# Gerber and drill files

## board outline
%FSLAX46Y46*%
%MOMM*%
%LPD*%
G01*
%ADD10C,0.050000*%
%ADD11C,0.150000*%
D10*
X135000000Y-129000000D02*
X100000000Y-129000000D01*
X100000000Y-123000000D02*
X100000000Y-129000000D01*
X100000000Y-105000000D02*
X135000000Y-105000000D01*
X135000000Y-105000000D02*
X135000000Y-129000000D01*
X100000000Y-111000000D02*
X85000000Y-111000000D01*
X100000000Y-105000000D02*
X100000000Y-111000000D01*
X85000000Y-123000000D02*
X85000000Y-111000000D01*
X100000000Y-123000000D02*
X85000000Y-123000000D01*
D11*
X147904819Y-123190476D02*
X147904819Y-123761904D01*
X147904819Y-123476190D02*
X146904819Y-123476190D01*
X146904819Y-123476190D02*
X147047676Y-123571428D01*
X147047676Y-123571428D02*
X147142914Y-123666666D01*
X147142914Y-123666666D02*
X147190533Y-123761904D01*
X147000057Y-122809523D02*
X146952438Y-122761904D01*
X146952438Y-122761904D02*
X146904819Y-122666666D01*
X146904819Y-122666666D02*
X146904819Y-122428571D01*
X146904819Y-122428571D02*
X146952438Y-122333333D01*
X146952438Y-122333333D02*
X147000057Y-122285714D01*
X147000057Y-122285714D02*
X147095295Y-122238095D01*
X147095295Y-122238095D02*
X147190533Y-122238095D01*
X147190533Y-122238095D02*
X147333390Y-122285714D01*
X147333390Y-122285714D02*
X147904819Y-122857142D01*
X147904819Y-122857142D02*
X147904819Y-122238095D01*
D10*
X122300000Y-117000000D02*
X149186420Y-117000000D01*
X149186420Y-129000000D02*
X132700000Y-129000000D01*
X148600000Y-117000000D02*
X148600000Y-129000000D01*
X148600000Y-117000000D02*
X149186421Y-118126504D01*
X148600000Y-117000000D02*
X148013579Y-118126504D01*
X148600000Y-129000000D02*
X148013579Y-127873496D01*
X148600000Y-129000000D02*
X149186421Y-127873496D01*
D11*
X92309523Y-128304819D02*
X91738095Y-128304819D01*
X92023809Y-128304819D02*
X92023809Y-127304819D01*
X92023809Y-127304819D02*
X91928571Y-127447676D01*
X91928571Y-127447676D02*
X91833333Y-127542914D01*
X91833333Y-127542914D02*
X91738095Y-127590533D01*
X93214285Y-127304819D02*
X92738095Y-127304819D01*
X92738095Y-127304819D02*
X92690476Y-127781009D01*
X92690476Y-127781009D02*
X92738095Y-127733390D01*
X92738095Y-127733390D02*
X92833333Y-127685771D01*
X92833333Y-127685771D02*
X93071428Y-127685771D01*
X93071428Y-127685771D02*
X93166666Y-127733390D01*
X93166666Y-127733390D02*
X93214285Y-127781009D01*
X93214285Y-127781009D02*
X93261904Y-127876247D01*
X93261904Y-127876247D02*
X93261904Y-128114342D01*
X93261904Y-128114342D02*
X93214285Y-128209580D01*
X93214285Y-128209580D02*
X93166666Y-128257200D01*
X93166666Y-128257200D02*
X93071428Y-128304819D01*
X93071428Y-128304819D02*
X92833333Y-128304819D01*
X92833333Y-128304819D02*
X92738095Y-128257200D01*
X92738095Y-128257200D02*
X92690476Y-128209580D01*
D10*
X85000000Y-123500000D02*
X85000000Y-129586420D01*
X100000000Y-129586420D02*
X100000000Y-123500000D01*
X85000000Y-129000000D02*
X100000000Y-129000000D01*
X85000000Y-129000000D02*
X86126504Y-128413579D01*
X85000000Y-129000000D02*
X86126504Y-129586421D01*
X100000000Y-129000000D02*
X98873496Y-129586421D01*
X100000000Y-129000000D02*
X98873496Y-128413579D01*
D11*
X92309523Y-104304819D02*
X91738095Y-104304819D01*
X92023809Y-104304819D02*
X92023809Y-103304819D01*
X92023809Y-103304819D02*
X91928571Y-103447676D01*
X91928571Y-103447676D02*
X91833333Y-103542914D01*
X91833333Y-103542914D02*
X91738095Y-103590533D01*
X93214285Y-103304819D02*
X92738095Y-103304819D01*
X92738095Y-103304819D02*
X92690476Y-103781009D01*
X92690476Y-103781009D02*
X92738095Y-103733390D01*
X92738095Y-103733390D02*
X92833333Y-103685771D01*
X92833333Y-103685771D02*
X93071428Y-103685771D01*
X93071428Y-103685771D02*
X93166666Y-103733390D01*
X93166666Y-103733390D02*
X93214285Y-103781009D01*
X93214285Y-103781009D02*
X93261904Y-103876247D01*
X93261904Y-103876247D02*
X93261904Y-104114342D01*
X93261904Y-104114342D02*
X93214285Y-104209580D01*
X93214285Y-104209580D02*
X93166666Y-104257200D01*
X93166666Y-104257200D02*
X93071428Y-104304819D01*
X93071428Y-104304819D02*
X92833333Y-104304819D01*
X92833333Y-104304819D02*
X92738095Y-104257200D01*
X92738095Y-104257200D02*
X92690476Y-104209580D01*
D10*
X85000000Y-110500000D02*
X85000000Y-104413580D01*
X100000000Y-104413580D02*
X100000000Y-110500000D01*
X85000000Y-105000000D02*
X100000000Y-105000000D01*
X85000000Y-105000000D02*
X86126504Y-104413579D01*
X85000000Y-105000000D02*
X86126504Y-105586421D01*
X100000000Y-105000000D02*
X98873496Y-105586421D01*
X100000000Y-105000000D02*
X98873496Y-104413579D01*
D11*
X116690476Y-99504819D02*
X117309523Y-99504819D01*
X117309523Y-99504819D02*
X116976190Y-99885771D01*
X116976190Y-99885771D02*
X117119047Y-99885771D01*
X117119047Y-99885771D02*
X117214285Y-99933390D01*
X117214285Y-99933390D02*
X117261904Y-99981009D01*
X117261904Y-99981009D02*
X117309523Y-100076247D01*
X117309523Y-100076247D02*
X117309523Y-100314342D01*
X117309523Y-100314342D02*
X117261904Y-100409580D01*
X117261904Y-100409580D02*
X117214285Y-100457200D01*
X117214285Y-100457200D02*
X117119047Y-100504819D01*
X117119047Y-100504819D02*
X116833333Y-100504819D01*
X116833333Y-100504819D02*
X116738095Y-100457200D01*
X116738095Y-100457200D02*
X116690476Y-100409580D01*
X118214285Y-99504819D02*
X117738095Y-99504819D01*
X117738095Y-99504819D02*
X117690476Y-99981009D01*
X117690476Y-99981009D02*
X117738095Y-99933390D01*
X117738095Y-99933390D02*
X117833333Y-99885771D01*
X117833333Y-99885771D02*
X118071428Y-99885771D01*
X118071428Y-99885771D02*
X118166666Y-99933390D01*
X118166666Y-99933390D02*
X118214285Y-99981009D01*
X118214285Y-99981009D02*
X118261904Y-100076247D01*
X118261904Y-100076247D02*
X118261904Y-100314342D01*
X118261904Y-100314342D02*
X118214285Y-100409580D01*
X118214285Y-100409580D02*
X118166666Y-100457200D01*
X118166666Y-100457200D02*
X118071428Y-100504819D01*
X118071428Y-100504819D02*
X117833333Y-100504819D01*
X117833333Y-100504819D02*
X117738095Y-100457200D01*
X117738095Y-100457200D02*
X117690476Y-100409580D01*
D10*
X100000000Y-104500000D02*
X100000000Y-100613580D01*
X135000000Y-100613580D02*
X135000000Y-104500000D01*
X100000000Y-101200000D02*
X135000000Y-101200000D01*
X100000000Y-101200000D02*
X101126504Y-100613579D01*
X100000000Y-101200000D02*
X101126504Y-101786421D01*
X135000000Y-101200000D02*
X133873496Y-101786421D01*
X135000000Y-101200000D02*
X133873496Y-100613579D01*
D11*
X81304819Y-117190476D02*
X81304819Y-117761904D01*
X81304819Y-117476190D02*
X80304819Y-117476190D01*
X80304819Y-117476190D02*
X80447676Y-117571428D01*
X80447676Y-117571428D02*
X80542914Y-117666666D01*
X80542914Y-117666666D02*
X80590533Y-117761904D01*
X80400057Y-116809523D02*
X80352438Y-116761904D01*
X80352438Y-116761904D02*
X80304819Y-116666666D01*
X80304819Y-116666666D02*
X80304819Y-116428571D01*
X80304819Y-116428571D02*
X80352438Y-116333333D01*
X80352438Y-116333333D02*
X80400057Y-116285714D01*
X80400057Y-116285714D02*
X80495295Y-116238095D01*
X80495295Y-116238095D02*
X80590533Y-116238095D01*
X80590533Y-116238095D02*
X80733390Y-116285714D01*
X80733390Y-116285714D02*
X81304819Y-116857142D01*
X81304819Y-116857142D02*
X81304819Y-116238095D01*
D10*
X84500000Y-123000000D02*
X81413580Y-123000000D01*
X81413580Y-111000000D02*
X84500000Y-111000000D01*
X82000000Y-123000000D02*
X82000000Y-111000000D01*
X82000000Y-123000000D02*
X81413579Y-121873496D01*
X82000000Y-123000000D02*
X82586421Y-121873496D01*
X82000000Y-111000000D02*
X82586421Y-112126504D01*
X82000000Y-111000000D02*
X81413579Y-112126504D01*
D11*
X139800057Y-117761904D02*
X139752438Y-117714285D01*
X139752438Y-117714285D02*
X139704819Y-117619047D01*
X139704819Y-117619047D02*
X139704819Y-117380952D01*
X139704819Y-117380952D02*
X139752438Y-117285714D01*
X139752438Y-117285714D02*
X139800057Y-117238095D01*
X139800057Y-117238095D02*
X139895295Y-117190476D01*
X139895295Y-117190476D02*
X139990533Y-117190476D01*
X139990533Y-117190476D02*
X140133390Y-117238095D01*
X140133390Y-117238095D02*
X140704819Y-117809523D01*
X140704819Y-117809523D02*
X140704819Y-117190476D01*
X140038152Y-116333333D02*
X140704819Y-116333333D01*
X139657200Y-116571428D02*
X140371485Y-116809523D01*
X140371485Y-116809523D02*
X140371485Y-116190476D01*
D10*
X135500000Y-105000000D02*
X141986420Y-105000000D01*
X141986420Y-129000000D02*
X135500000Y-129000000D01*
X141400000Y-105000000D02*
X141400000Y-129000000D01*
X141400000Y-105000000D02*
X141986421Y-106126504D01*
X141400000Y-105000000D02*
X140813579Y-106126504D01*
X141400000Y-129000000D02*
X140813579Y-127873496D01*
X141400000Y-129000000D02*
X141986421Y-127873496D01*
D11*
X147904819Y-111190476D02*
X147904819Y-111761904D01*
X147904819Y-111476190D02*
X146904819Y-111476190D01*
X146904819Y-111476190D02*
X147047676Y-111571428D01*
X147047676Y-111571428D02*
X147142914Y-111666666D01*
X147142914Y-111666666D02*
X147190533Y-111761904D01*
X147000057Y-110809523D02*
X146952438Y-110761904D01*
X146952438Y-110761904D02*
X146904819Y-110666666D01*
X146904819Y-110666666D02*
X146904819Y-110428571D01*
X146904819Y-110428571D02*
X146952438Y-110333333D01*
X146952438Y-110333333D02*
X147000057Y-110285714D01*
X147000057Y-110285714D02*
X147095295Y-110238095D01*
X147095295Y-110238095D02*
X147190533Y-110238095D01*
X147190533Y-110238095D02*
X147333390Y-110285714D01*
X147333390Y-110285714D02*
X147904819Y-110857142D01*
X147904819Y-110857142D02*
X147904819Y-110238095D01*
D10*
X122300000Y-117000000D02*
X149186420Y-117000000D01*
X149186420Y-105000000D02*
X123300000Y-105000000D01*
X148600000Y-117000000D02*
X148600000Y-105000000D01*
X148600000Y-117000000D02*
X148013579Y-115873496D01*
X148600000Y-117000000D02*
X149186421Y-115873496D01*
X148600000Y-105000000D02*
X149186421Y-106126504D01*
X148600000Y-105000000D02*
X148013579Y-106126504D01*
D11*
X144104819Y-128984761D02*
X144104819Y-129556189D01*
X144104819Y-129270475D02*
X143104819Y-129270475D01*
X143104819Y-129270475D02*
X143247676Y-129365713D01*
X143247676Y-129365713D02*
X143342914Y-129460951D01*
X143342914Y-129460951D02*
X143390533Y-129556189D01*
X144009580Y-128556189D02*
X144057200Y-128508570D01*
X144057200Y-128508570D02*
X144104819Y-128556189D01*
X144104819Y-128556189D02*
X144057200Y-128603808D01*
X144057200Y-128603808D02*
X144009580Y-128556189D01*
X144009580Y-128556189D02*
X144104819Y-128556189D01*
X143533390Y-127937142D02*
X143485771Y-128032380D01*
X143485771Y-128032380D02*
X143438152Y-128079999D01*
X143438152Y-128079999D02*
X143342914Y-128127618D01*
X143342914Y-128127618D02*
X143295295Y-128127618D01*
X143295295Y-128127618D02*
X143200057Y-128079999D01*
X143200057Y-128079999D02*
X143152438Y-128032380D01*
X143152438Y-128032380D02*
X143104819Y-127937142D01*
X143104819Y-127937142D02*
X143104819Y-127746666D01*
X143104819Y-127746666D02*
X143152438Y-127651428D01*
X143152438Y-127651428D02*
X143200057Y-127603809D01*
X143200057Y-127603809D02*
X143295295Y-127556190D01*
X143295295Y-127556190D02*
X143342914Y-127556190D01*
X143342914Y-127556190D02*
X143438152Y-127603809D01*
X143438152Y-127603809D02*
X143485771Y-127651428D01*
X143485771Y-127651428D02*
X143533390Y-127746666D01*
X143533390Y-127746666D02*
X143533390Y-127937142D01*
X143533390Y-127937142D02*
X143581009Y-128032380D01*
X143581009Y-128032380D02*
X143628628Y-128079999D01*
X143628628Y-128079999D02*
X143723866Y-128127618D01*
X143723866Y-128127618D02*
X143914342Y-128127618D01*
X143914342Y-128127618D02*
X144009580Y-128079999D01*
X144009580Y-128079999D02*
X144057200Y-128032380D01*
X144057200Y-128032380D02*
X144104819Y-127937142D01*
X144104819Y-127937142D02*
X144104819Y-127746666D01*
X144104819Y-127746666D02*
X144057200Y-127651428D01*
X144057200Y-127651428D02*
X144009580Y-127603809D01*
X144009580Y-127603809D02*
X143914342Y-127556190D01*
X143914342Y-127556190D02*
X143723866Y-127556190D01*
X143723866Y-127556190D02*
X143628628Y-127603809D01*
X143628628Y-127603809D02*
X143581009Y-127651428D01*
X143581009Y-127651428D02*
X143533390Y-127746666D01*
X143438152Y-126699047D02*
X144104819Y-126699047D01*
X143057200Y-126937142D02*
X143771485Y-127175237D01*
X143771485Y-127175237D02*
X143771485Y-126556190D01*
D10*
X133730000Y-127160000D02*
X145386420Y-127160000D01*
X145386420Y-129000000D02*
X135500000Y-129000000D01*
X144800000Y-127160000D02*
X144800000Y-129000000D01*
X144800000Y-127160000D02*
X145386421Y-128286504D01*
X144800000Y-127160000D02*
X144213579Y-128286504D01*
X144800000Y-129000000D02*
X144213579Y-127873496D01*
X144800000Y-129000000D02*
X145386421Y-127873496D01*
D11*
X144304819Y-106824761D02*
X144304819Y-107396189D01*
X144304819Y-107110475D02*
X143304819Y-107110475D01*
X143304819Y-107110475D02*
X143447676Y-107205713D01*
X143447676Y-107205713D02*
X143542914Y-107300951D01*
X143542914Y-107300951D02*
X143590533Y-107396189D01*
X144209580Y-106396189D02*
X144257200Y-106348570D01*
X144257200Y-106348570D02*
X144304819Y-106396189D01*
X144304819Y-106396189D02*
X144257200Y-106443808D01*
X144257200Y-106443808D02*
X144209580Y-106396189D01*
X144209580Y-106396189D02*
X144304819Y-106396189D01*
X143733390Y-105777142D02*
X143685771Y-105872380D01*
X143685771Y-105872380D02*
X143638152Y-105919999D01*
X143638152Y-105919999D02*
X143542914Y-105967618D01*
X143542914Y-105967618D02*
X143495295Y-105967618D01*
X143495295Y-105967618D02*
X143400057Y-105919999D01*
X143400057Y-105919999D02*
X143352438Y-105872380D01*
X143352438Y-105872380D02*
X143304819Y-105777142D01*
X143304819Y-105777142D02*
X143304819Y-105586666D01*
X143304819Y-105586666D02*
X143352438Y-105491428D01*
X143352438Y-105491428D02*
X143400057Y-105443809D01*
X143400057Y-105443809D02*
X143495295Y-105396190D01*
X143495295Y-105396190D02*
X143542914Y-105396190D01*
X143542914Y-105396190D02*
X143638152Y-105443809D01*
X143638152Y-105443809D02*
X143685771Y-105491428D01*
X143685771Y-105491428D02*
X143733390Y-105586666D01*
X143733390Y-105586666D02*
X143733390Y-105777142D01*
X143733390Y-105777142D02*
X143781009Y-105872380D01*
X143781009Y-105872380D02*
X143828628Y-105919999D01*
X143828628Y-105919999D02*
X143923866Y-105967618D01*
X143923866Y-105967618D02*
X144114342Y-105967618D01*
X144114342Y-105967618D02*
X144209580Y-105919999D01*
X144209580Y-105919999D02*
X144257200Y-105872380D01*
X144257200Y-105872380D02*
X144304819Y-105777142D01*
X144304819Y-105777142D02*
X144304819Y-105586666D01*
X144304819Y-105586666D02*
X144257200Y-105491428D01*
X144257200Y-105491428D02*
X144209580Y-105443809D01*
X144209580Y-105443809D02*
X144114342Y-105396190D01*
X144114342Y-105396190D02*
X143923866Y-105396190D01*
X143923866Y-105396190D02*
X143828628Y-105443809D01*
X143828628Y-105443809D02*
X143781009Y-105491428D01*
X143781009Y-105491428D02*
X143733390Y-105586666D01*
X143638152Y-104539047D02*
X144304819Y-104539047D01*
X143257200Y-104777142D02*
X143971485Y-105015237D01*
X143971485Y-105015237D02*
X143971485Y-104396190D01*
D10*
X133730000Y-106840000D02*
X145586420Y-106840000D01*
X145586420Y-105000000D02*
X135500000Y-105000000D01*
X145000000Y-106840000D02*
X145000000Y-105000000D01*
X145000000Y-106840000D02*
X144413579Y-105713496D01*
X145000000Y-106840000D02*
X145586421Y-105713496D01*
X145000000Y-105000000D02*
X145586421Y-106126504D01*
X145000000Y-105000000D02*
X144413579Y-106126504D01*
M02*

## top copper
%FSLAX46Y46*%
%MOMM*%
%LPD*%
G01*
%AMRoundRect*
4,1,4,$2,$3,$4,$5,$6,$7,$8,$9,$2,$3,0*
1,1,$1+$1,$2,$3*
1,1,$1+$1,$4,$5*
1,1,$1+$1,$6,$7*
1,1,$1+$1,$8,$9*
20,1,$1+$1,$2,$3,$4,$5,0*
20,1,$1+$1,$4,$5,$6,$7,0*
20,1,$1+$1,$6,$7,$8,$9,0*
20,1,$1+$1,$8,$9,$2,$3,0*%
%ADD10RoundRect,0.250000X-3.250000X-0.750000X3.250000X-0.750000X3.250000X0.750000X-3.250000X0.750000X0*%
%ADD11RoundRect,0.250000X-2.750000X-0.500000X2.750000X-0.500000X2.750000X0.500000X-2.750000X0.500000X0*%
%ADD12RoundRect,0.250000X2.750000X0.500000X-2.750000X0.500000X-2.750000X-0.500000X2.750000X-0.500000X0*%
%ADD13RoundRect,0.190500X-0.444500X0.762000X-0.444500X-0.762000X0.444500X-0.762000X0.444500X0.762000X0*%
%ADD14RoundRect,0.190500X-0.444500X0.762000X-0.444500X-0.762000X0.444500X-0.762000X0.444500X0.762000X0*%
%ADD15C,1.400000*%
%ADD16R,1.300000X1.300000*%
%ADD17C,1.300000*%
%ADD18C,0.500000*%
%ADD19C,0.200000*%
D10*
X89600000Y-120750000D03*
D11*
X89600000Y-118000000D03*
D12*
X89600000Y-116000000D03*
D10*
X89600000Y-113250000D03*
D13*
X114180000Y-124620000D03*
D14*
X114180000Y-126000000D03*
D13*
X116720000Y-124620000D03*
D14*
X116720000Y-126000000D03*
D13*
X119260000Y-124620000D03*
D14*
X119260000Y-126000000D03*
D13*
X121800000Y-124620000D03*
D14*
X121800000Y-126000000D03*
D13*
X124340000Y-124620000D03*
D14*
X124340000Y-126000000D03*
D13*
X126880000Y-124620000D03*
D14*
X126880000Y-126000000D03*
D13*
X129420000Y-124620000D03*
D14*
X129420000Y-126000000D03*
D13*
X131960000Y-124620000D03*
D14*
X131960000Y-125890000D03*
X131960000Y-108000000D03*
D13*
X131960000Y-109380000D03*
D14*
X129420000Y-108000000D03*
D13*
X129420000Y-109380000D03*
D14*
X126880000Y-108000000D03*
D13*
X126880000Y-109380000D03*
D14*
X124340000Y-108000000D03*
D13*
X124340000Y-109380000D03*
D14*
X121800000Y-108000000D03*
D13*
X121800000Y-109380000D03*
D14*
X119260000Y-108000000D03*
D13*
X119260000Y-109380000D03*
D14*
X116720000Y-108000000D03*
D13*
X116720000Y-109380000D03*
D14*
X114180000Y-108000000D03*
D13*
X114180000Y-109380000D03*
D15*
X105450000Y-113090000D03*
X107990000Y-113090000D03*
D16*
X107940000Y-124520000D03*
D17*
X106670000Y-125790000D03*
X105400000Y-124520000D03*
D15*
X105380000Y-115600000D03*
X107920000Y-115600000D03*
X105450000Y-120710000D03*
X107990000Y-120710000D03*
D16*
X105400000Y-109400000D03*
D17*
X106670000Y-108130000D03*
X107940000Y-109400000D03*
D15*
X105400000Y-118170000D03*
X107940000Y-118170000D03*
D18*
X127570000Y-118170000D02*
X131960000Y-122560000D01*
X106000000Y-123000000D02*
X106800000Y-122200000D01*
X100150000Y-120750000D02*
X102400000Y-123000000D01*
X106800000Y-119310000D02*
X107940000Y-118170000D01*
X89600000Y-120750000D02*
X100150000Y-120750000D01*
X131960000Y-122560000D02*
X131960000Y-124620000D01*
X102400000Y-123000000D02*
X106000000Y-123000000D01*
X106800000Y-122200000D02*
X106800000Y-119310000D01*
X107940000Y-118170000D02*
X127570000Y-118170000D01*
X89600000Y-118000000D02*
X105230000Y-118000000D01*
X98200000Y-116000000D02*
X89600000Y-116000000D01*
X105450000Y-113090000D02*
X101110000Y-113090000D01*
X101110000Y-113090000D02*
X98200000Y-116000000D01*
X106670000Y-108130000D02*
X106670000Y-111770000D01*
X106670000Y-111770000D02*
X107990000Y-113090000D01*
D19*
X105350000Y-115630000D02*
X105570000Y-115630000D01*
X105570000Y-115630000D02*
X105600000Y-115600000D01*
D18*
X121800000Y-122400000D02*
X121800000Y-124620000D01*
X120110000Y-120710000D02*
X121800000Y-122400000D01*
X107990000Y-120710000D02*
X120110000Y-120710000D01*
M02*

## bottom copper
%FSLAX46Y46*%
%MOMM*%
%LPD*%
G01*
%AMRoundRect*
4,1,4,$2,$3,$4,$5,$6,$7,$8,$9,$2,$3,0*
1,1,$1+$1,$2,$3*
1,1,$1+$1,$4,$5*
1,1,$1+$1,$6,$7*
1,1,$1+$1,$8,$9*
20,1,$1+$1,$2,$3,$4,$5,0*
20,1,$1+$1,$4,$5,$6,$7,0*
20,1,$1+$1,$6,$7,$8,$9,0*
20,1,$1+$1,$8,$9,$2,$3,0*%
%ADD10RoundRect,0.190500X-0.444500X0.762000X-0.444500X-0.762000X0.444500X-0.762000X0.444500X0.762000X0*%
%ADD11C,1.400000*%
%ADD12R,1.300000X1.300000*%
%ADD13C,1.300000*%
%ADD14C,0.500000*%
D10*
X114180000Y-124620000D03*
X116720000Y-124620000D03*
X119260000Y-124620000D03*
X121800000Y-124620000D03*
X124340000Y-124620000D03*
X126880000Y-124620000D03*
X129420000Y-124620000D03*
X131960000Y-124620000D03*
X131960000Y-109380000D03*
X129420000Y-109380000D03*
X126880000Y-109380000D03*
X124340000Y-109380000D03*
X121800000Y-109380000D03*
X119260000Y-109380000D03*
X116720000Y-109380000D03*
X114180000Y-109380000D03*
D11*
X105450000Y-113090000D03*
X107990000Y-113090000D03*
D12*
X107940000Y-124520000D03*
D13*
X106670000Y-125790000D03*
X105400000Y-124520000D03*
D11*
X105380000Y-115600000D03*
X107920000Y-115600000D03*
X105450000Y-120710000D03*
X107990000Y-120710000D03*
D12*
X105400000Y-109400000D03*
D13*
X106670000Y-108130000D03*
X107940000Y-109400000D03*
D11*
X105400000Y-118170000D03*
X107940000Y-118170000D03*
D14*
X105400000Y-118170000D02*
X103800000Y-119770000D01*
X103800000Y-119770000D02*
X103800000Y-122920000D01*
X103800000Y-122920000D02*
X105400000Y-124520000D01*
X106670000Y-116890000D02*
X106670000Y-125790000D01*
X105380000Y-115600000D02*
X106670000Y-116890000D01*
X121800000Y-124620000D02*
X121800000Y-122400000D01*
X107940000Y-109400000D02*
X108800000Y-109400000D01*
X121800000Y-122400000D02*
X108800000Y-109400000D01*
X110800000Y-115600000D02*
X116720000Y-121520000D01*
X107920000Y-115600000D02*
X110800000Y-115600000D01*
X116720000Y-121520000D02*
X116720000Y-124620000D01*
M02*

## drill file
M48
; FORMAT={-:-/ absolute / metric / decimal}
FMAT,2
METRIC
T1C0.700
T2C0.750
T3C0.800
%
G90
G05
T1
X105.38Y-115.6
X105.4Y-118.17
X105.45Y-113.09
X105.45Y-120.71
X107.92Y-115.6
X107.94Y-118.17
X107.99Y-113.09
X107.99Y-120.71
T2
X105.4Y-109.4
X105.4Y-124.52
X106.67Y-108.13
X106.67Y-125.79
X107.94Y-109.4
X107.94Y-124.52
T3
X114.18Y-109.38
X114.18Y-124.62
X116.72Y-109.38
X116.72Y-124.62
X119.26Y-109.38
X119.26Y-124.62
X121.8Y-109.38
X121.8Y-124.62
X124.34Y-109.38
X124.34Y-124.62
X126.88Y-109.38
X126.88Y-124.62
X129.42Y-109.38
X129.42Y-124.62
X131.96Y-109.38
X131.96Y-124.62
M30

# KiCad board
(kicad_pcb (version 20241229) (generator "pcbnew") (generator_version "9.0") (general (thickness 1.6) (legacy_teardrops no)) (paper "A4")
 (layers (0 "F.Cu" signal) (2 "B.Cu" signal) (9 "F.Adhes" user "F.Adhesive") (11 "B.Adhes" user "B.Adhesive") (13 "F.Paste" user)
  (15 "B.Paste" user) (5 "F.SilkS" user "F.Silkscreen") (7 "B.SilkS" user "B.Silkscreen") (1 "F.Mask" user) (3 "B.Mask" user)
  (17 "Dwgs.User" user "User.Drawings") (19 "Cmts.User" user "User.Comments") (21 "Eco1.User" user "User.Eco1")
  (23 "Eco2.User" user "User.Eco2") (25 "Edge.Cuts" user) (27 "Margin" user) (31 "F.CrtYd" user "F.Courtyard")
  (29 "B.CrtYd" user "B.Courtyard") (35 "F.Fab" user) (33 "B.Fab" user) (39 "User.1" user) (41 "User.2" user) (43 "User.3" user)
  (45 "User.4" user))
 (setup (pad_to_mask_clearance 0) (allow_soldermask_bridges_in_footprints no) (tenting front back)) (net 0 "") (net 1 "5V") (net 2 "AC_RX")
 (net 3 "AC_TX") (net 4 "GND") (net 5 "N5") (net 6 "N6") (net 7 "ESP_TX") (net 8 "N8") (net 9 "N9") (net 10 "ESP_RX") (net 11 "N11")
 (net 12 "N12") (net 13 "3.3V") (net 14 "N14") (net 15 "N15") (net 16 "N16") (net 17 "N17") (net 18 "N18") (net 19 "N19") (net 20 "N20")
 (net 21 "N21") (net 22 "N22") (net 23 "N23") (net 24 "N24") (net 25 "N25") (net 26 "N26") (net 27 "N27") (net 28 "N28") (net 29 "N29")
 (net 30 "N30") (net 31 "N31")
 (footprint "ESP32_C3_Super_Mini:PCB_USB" (layer "F.Cu") (at 89.6 117)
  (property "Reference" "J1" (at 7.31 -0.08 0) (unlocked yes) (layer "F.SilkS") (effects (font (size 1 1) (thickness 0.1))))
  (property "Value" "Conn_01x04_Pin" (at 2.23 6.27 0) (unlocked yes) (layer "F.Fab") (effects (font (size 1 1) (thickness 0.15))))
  (pad "1" smd roundrect (at 0 3.75) (size 7 2) (layers "F.Cu" "F.Mask" "F.Paste") (roundrect_rratio 0.125) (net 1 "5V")
   (thermal_bridge_angle 45))
  (pad "2" smd roundrect (at 0 1) (size 6 1.5) (layers "F.Cu" "F.Mask" "F.Paste") (roundrect_rratio 0.1666666667) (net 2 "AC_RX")
   (thermal_bridge_angle 45))
  (pad "3" smd roundrect (at 0 -1 180) (size 6 1.5) (layers "F.Cu" "F.Mask" "F.Paste") (roundrect_rratio 0.1666666667) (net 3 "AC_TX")
   (thermal_bridge_angle 45))
  (pad "4" smd roundrect (at 0 -3.75) (size 7 2) (layers "F.Cu" "F.Mask" "F.Paste") (roundrect_rratio 0.125) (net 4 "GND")
   (thermal_bridge_angle 45)))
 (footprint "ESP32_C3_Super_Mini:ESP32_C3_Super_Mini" (layer "F.Cu") (at 121.8 117 -90)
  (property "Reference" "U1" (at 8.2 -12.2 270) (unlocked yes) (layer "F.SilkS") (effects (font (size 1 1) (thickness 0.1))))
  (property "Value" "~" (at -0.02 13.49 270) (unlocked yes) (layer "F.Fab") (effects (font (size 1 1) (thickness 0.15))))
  (pad "0" thru_hole roundrect (at 7.62 7.62 270) (size 1.905 1.27) (drill 0.8) (layers "*.Cu" "*.Mask") (remove_unused_layers no)
   (roundrect_rratio 0.15) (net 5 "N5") (thermal_bridge_angle 45))
  (pad "0" smd roundrect (at 9 7.62 270) (size 1.905 1.27) (layers "F.Cu" "F.Mask" "F.Paste") (roundrect_rratio 0.15) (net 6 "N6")
   (thermal_bridge_angle 45))
  (pad "1" thru_hole roundrect (at 7.62 5.08 270) (size 1.905 1.27) (drill 0.8) (layers "*.Cu" "*.Mask") (remove_unused_layers no)
   (roundrect_rratio 0.15) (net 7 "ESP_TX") (thermal_bridge_angle 45))
  (pad "1" smd roundrect (at 9 5.08 270) (size 1.905 1.27) (layers "F.Cu" "F.Mask" "F.Paste") (roundrect_rratio 0.15) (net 7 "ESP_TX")
   (thermal_bridge_angle 45))
  (pad "2" thru_hole roundrect (at 7.62 2.54 270) (size 1.905 1.27) (drill 0.8) (layers "*.Cu" "*.Mask") (remove_unused_layers no)
   (roundrect_rratio 0.15) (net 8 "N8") (thermal_bridge_angle 45))
  (pad "2" smd roundrect (at 9 2.54 270) (size 1.905 1.27) (layers "F.Cu" "F.Mask" "F.Paste") (roundrect_rratio 0.15) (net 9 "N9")
   (thermal_bridge_angle 45))
  (pad "3" thru_hole roundrect (at 7.62 0 270) (size 1.905 1.27) (drill 0.8) (layers "*.Cu" "*.Mask") (remove_unused_layers no)
   (roundrect_rratio 0.15) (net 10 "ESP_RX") (thermal_bridge_angle 45))
  (pad "3" smd roundrect (at 9 0 270) (size 1.905 1.27) (layers "F.Cu" "F.Mask" "F.Paste") (roundrect_rratio 0.15) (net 10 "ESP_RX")
   (thermal_bridge_angle 45))
  (pad "4" thru_hole roundrect (at 7.62 -2.54 270) (size 1.905 1.27) (drill 0.8) (layers "*.Cu" "*.Mask") (remove_unused_layers no)
   (roundrect_rratio 0.15) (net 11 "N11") (thermal_bridge_angle 45))
  (pad "4" smd roundrect (at 9 -2.54 270) (size 1.905 1.27) (layers "F.Cu" "F.Mask" "F.Paste") (roundrect_rratio 0.15) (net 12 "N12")
   (thermal_bridge_angle 45))
  (pad "5" thru_hole roundrect (at 7.62 -5.08 270) (size 1.905 1.27) (drill 0.8) (layers "*.Cu" "*.Mask") (remove_unused_layers no)
   (roundrect_rratio 0.15) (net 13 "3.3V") (thermal_bridge_angle 45))
  (pad "5" smd roundrect (at 9 -5.08 270) (size 1.905 1.27) (layers "F.Cu" "F.Mask" "F.Paste") (roundrect_rratio 0.15) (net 13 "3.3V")
   (thermal_bridge_angle 45))
  (pad "6" thru_hole roundrect (at 7.62 -7.62 270) (size 1.905 1.27) (drill 0.8) (layers "*.Cu" "*.Mask") (remove_unused_layers no)
   (roundrect_rratio 0.15) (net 4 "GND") (thermal_bridge_angle 45))
  (pad "6" smd roundrect (at 9 -7.62 270) (size 1.905 1.27) (layers "F.Cu" "F.Mask" "F.Paste") (roundrect_rratio 0.15) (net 4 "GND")
   (thermal_bridge_angle 45))
  (pad "7" thru_hole roundrect (at 7.62 -10.16 270) (size 1.905 1.27) (drill 0.8) (layers "*.Cu" "*.Mask") (remove_unused_layers no)
   (roundrect_rratio 0.15) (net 1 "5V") (thermal_bridge_angle 45))
  (pad "7" smd roundrect (at 8.89 -10.16 270) (size 1.905 1.27) (layers "F.Cu" "F.Mask" "F.Paste") (roundrect_rratio 0.15) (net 1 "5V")
   (thermal_bridge_angle 45))
  (pad "8" smd roundrect (at -9 -10.16 270) (size 1.905 1.27) (layers "F.Cu" "F.Mask" "F.Paste") (roundrect_rratio 0.15) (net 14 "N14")
   (thermal_bridge_angle 45))
  (pad "8" thru_hole roundrect (at -7.62 -10.16 270) (size 1.905 1.27) (drill 0.8) (layers "*.Cu" "*.Mask") (remove_unused_layers no)
   (roundrect_rratio 0.15) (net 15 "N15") (thermal_bridge_angle 45))
  (pad "9" smd roundrect (at -9 -7.62 270) (size 1.905 1.27) (layers "F.Cu" "F.Mask" "F.Paste") (roundrect_rratio 0.15) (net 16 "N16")
   (thermal_bridge_angle 45))
  (pad "9" thru_hole roundrect (at -7.62 -7.62 270) (size 1.905 1.27) (drill 0.8) (layers "*.Cu" "*.Mask") (remove_unused_layers no)
   (roundrect_rratio 0.15) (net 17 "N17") (thermal_bridge_angle 45))
  (pad "10" smd roundrect (at -9 -5.08 270) (size 1.905 1.27) (layers "F.Cu" "F.Mask" "F.Paste") (roundrect_rratio 0.15) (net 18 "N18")
   (thermal_bridge_angle 45))
  (pad "10" thru_hole roundrect (at -7.62 -5.08 270) (size 1.905 1.27) (drill 0.8) (layers "*.Cu" "*.Mask") (remove_unused_layers no)
   (roundrect_rratio 0.15) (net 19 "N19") (thermal_bridge_angle 45))
  (pad "11" smd roundrect (at -9 -2.54 270) (size 1.905 1.27) (layers "F.Cu" "F.Mask" "F.Paste") (roundrect_rratio 0.15) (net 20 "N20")
   (thermal_bridge_angle 45))
  (pad "11" thru_hole roundrect (at -7.62 -2.54 270) (size 1.905 1.27) (drill 0.8) (layers "*.Cu" "*.Mask") (remove_unused_layers no)
   (roundrect_rratio 0.15) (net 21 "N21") (thermal_bridge_angle 45))
  (pad "12" smd roundrect (at -9 0 270) (size 1.905 1.27) (layers "F.Cu" "F.Mask" "F.Paste") (roundrect_rratio 0.15) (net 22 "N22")
   (thermal_bridge_angle 45))
  (pad "12" thru_hole roundrect (at -7.62 0 270) (size 1.905 1.27) (drill 0.8) (layers "*.Cu" "*.Mask") (remove_unused_layers no)
   (roundrect_rratio 0.15) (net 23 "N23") (thermal_bridge_angle 45))
  (pad "13" smd roundrect (at -9 2.54 270) (size 1.905 1.27) (layers "F.Cu" "F.Mask" "F.Paste") (roundrect_rratio 0.15) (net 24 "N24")
   (thermal_bridge_angle 45))
  (pad "13" thru_hole roundrect (at -7.62 2.54 270) (size 1.905 1.27) (drill 0.8) (layers "*.Cu" "*.Mask") (remove_unused_layers no)
   (roundrect_rratio 0.15) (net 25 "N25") (thermal_bridge_angle 45))
  (pad "14" smd roundrect (at -9 5.08 270) (size 1.905 1.27) (layers "F.Cu" "F.Mask" "F.Paste") (roundrect_rratio 0.15) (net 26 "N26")
   (thermal_bridge_angle 45))
  (pad "14" thru_hole roundrect (at -7.62 5.08 270) (size 1.905 1.27) (drill 0.8) (layers "*.Cu" "*.Mask") (remove_unused_layers no)
   (roundrect_rratio 0.15) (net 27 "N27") (thermal_bridge_angle 45))
  (pad "15" smd roundrect (at -9 7.62 270) (size 1.905 1.27) (layers "F.Cu" "F.Mask" "F.Paste") (roundrect_rratio 0.15) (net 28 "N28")
   (thermal_bridge_angle 45))
  (pad "15" thru_hole roundrect (at -7.62 7.62 270) (size 1.905 1.27) (drill 0.8) (layers "*.Cu" "*.Mask") (remove_unused_layers no)
   (roundrect_rratio 0.15) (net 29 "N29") (thermal_bridge_angle 45)))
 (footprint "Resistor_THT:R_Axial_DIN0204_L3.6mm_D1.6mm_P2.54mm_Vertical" (layer "F.Cu") (at 105.45 113.09)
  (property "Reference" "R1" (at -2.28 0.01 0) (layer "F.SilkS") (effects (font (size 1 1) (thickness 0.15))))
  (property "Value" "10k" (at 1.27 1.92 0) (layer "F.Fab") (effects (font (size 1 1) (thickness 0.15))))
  (pad "1" thru_hole circle (at 0 0) (size 1.4 1.4) (drill 0.7) (layers "*.Cu" "*.Mask") (remove_unused_layers no) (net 3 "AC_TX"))
  (pad "2" thru_hole circle (at 2.54 0) (size 1.4 1.4) (drill 0.7) (layers "*.Cu" "*.Mask") (remove_unused_layers no) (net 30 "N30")))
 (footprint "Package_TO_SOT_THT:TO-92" (layer "F.Cu") (at 107.94 124.52 180)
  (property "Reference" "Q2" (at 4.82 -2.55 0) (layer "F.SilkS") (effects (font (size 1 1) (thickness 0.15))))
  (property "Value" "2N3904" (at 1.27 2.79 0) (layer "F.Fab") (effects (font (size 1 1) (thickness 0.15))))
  (pad "1" thru_hole rect (at 0 0 180) (size 1.3 1.3) (drill 0.75) (layers "*.Cu" "*.Mask") (remove_unused_layers no) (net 4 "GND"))
  (pad "2" thru_hole circle (at 1.27 -1.27 180) (size 1.3 1.3) (drill 0.75) (layers "*.Cu" "*.Mask") (remove_unused_layers no)
   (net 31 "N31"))
  (pad "3" thru_hole circle (at 2.54 0 180) (size 1.3 1.3) (drill 0.75) (layers "*.Cu" "*.Mask") (remove_unused_layers no) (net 2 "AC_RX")))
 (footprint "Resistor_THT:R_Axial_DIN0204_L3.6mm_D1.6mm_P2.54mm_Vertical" (layer "F.Cu") (at 105.38 115.6)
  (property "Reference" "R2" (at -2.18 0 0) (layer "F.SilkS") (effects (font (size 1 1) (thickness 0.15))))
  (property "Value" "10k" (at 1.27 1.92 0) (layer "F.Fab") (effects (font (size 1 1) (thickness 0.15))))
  (pad "1" thru_hole circle (at 0 0) (size 1.4 1.4) (drill 0.7) (layers "*.Cu" "*.Mask") (remove_unused_layers no) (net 31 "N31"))
  (pad "2" thru_hole circle (at 2.54 0) (size 1.4 1.4) (drill 0.7) (layers "*.Cu" "*.Mask") (remove_unused_layers no) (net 7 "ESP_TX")))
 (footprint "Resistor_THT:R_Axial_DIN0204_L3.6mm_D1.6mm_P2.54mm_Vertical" (layer "F.Cu") (at 105.45 120.71)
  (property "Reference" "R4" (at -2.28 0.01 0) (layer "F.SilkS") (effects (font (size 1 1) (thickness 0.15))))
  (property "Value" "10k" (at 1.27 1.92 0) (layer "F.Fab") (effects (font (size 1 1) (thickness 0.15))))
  (pad "1" thru_hole circle (at 0 0) (size 1.4 1.4) (drill 0.7) (layers "*.Cu" "*.Mask") (remove_unused_layers no) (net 13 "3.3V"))
  (pad "2" thru_hole circle (at 2.54 0) (size 1.4 1.4) (drill 0.7) (layers "*.Cu" "*.Mask") (remove_unused_layers no) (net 10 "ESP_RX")))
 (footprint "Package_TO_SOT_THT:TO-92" (layer "F.Cu") (at 105.4 109.4)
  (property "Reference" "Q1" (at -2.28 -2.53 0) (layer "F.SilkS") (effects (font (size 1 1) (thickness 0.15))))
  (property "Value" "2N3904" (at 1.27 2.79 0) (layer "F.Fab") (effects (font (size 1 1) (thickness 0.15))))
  (pad "1" thru_hole rect (at 0 0) (size 1.3 1.3) (drill 0.75) (layers "*.Cu" "*.Mask") (remove_unused_layers no) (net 4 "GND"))
  (pad "2" thru_hole circle (at 1.27 -1.27) (size 1.3 1.3) (drill 0.75) (layers "*.Cu" "*.Mask") (remove_unused_layers no) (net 30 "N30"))
  (pad "3" thru_hole circle (at 2.54 0) (size 1.3 1.3) (drill 0.75) (layers "*.Cu" "*.Mask") (remove_unused_layers no) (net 10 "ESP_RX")))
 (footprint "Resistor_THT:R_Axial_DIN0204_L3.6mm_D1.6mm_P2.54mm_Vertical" (layer "F.Cu") (at 105.4 118.17)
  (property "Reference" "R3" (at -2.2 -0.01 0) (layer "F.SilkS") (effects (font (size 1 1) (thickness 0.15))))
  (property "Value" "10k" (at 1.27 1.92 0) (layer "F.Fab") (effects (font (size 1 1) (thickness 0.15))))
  (pad "1" thru_hole circle (at 0 0) (size 1.4 1.4) (drill 0.7) (layers "*.Cu" "*.Mask") (remove_unused_layers no) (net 2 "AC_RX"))
  (pad "2" thru_hole circle (at 2.54 0) (size 1.4 1.4) (drill 0.7) (layers "*.Cu" "*.Mask") (remove_unused_layers no) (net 1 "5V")))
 (gr_line (start 135 129) (end 100 129) (stroke (width 0.05) (type solid)) (layer "Edge.Cuts"))
 (gr_line (start 100 123) (end 100 129) (stroke (width 0.05) (type default)) (layer "Edge.Cuts"))
 (gr_line (start 100 105) (end 135 105) (stroke (width 0.05) (type default)) (layer "Edge.Cuts"))
 (gr_line (start 135 105) (end 135 129) (stroke (width 0.05) (type default)) (layer "Edge.Cuts"))
 (gr_line (start 100 111) (end 85 111) (stroke (width 0.05) (type solid)) (layer "Edge.Cuts"))
 (gr_line (start 100 105) (end 100 111) (stroke (width 0.05) (type default)) (layer "Edge.Cuts"))
 (gr_line (start 85 123) (end 85 111) (stroke (width 0.05) (type default)) (layer "Edge.Cuts"))
 (gr_line (start 100 123) (end 85 123) (stroke (width 0.05) (type default)) (layer "Edge.Cuts"))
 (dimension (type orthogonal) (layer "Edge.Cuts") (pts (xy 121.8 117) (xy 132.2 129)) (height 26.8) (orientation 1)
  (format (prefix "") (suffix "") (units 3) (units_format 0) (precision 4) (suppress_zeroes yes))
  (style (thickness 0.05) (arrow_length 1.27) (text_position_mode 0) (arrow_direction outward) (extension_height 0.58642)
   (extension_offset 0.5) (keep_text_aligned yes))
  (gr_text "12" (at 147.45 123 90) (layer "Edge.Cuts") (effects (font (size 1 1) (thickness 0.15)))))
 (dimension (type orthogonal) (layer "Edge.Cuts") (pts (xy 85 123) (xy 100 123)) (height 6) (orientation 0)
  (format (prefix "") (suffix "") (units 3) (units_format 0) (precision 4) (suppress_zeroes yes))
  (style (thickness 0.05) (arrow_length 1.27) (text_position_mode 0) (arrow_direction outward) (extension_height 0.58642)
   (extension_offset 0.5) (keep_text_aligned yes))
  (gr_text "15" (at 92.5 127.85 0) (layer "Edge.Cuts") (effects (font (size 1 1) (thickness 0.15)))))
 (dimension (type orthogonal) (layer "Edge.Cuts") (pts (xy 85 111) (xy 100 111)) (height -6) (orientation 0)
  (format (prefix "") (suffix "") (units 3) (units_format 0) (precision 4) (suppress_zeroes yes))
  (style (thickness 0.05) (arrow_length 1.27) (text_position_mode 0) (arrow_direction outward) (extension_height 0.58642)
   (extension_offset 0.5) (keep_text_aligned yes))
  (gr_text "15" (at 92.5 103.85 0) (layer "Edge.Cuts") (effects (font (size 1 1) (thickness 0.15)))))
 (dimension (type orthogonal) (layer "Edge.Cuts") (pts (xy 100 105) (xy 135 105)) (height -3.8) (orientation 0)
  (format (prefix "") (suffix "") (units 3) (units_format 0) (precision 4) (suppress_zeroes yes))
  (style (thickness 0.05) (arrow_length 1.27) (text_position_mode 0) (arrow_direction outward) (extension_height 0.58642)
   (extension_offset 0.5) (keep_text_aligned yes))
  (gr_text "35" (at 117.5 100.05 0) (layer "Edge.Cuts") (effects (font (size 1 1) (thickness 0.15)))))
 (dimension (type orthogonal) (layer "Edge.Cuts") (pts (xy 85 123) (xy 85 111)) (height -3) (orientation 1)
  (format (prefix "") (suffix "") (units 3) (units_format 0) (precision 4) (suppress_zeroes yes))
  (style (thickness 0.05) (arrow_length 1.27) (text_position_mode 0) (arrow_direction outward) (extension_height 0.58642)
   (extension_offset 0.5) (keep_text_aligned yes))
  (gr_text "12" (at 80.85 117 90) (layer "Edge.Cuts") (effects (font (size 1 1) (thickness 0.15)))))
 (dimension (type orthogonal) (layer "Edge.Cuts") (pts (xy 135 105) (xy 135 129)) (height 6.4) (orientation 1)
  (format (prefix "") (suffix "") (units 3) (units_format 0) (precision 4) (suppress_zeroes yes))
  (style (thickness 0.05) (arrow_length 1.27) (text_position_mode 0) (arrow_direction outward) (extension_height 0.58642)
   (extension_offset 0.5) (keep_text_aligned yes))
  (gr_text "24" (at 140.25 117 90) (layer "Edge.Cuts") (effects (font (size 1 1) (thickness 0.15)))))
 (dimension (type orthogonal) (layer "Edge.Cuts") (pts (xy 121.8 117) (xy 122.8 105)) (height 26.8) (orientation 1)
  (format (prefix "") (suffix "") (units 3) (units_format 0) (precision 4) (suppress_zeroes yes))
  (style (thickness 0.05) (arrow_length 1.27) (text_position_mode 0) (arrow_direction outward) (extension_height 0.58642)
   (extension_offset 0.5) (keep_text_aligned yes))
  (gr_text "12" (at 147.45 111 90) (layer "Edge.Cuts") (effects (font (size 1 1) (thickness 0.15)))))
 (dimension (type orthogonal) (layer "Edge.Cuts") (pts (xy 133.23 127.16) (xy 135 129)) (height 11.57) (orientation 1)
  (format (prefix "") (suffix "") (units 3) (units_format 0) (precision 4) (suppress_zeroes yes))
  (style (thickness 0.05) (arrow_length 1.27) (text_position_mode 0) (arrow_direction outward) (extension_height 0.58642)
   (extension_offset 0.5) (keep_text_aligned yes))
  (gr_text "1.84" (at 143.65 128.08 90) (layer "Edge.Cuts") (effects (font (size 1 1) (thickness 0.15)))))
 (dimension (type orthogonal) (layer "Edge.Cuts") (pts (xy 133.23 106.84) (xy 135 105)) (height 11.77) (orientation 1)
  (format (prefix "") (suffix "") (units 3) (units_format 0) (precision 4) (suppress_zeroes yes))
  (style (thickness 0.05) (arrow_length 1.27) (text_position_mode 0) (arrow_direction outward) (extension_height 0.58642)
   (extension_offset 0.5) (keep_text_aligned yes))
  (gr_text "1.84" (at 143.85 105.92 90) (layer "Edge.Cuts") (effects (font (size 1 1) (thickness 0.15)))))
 (segment (start 127.57 118.17) (end 131.96 122.56) (width 0.5) (layer "F.Cu") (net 1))
 (segment (start 106 123) (end 106.8 122.2) (width 0.5) (layer "F.Cu") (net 1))
 (segment (start 100.15 120.75) (end 102.4 123) (width 0.5) (layer "F.Cu") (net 1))
 (segment (start 106.8 119.31) (end 107.94 118.17) (width 0.5) (layer "F.Cu") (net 1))
 (segment (start 89.6 120.75) (end 100.15 120.75) (width 0.5) (layer "F.Cu") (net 1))
 (segment (start 131.96 122.56) (end 131.96 124.62) (width 0.5) (layer "F.Cu") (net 1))
 (segment (start 102.4 123) (end 106 123) (width 0.5) (layer "F.Cu") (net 1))
 (segment (start 106.8 122.2) (end 106.8 119.31) (width 0.5) (layer "F.Cu") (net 1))
 (segment (start 107.94 118.17) (end 127.57 118.17) (width 0.5) (layer "F.Cu") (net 1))
 (segment (start 89.6 118) (end 105.23 118) (width 0.5) (layer "F.Cu") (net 2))
 (segment (start 105.4 118.17) (end 103.8 119.77) (width 0.5) (layer "B.Cu") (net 2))
 (segment (start 103.8 119.77) (end 103.8 122.92) (width 0.5) (layer "B.Cu") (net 2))
 (segment (start 103.8 122.92) (end 105.4 124.52) (width 0.5) (layer "B.Cu") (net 2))
 (segment (start 98.2 116) (end 89.6 116) (width 0.5) (layer "F.Cu") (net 3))
 (segment (start 105.45 113.09) (end 101.11 113.09) (width 0.5) (layer "F.Cu") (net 3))
 (segment (start 101.11 113.09) (end 98.2 116) (width 0.5) (layer "F.Cu") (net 3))
 (segment (start 106.67 108.13) (end 106.67 111.77) (width 0.5) (layer "F.Cu") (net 30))
 (segment (start 106.67 111.77) (end 107.99 113.09) (width 0.5) (layer "F.Cu") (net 30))
 (segment (start 105.35 115.63) (end 105.57 115.63) (width 0.2) (layer "F.Cu") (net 31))
 (segment (start 105.57 115.63) (end 105.6 115.6) (width 0.2) (layer "F.Cu") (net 31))
 (segment (start 106.67 116.89) (end 106.67 125.79) (width 0.5) (layer "B.Cu") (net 31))
 (segment (start 105.38 115.6) (end 106.67 116.89) (width 0.5) (layer "B.Cu") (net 31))
 (segment (start 121.8 122.4) (end 121.8 124.62) (width 0.5) (layer "F.Cu") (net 10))
 (segment (start 120.11 120.71) (end 121.8 122.4) (width 0.5) (layer "F.Cu") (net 10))
 (segment (start 107.99 120.71) (end 120.11 120.71) (width 0.5) (layer "F.Cu") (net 10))
 (segment (start 121.8 124.62) (end 121.8 122.4) (width 0.5) (layer "B.Cu") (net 10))
 (segment (start 107.94 109.4) (end 108.8 109.4) (width 0.5) (layer "B.Cu") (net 10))
 (segment (start 121.8 122.4) (end 108.8 109.4) (width 0.5) (layer "B.Cu") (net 10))
 (segment (start 110.8 115.6) (end 116.72 121.52) (width 0.5) (layer "B.Cu") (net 7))
 (segment (start 107.92 115.6) (end 110.8 115.6) (width 0.5) (layer "B.Cu") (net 7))
 (segment (start 116.72 121.52) (end 116.72 124.62) (width 0.5) (layer "B.Cu") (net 7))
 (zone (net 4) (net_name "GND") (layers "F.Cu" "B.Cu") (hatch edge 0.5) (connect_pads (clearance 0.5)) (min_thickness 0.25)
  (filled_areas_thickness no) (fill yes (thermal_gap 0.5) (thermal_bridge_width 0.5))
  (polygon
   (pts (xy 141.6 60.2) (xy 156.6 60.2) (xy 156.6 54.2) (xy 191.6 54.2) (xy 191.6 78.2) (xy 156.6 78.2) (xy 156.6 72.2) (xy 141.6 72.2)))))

